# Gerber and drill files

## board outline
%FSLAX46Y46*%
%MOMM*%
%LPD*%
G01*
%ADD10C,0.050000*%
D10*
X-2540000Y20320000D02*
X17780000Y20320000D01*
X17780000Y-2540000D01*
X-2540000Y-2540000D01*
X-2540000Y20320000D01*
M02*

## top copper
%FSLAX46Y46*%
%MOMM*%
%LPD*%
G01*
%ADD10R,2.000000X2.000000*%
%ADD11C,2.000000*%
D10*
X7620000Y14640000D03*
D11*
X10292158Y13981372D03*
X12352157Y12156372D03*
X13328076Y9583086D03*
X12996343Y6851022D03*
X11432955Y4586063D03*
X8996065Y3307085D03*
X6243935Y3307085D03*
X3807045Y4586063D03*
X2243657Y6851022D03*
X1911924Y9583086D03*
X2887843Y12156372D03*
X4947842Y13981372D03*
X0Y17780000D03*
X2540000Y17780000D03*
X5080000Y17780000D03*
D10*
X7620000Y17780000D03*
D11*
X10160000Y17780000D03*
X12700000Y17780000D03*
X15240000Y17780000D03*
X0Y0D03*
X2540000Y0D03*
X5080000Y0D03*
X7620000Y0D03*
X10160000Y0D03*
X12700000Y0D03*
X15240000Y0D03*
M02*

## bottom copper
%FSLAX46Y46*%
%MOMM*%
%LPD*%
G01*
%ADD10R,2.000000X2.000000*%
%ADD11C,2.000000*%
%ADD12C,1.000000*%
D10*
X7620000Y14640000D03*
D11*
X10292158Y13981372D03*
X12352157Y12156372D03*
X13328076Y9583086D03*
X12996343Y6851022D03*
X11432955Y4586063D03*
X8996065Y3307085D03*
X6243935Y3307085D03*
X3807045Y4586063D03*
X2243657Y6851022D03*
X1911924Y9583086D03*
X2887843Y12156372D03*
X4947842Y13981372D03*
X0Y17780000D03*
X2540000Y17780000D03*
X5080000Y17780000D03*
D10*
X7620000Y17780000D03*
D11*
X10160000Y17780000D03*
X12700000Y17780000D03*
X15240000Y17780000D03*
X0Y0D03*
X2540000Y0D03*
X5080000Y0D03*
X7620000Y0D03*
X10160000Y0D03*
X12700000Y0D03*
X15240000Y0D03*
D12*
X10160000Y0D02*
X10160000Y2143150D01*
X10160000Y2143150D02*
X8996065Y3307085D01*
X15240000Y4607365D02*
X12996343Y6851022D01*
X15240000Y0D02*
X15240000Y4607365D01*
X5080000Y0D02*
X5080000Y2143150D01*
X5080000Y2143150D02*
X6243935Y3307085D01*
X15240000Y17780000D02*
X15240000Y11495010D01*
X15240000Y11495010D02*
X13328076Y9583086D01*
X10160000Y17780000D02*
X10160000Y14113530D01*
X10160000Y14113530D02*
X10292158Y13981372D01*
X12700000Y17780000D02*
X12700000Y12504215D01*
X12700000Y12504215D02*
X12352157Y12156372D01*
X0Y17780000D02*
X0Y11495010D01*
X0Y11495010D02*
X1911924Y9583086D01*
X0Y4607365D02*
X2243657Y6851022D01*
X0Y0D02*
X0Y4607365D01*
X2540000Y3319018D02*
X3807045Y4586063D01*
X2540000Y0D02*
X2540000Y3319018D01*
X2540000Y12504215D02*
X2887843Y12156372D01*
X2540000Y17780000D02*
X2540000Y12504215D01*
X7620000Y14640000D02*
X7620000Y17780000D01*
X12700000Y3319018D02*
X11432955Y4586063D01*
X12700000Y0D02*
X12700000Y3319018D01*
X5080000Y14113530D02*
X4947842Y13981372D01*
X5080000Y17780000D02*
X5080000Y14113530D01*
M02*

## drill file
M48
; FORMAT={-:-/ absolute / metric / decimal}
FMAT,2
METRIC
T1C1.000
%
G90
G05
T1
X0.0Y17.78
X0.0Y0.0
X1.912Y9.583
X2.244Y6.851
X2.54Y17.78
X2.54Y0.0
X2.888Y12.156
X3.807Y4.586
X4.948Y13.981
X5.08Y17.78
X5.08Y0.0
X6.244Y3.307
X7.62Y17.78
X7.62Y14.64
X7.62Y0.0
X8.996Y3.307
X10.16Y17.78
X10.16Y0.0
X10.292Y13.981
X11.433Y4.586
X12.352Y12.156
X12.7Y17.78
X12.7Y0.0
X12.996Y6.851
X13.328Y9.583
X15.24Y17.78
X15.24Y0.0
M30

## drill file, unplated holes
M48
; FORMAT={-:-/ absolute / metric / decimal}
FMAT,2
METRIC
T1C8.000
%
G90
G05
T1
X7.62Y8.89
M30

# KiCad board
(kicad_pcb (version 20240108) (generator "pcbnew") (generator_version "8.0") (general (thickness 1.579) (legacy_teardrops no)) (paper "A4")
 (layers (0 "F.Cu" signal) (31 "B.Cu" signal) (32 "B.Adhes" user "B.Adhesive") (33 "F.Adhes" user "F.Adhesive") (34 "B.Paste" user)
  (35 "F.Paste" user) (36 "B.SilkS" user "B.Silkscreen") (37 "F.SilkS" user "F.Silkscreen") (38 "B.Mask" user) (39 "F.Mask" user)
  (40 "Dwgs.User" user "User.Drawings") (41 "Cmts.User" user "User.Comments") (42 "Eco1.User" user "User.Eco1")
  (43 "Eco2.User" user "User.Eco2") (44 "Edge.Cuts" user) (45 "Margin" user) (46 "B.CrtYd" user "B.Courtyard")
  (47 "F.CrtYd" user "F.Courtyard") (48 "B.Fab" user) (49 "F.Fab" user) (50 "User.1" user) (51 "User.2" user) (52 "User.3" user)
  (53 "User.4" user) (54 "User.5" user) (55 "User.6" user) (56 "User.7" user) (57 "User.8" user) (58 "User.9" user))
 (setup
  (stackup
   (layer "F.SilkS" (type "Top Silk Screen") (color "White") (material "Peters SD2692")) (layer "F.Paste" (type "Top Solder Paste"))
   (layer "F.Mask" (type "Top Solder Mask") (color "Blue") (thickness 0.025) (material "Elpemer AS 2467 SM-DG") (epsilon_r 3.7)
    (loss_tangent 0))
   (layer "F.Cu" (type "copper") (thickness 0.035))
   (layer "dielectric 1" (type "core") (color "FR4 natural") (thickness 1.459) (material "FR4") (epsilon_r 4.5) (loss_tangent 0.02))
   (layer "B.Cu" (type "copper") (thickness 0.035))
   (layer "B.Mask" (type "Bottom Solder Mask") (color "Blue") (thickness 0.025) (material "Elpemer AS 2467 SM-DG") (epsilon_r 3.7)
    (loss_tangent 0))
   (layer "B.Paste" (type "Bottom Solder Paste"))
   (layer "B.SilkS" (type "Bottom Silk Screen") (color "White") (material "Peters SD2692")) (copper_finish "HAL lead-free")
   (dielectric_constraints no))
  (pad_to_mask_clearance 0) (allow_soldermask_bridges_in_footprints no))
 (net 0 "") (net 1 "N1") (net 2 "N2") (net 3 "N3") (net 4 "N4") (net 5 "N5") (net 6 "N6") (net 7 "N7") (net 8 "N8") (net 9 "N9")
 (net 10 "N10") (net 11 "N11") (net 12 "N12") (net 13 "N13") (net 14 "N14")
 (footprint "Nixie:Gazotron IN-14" (layer "F.Cu") (at 7.62 -8.89)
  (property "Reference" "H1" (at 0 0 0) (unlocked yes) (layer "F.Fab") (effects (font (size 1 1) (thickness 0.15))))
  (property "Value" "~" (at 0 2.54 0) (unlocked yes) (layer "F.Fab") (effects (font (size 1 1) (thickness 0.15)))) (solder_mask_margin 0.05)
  (pad "" np_thru_hole circle (at 0 0) (size 2 2) (drill 8) (layers "*.Mask"))
  (pad "1" thru_hole rect (at 0 -5.75) (size 2 2) (drill 1) (layers "*.Cu" "B.Mask") (remove_unused_layers no) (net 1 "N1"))
  (pad "2" thru_hole circle (at 2.672158 -5.091372) (size 2 2) (drill 1) (layers "*.Cu" "B.Mask") (remove_unused_layers no) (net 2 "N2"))
  (pad "3" thru_hole circle (at 4.732157 -3.266372) (size 2 2) (drill 1) (layers "*.Cu" "B.Mask") (remove_unused_layers no) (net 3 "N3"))
  (pad "4" thru_hole circle (at 5.708076 -0.693086) (size 2 2) (drill 1) (layers "*.Cu" "B.Mask") (remove_unused_layers no) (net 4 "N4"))
  (pad "5" thru_hole circle (at 5.376343 2.038978) (size 2 2) (drill 1) (layers "*.Cu" "B.Mask") (remove_unused_layers no) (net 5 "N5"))
  (pad "6" thru_hole circle (at 3.812955 4.303937) (size 2 2) (drill 1) (layers "*.Cu" "B.Mask") (remove_unused_layers no) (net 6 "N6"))
  (pad "7" thru_hole circle (at 1.376065 5.582915) (size 2 2) (drill 1) (layers "*.Cu" "B.Mask") (remove_unused_layers no) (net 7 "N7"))
  (pad "8" thru_hole circle (at -1.376065 5.582915) (size 2 2) (drill 1) (layers "*.Cu" "B.Mask") (remove_unused_layers no) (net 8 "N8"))
  (pad "9" thru_hole circle (at -3.812955 4.303937) (size 2 2) (drill 1) (layers "*.Cu" "B.Mask") (remove_unused_layers no) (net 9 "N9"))
  (pad "10" thru_hole circle (at -5.376343 2.038978) (size 2 2) (drill 1) (layers "*.Cu" "B.Mask") (remove_unused_layers no) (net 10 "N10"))
  (pad "11" thru_hole circle (at -5.708076 -0.693086) (size 2 2) (drill 1) (layers "*.Cu" "B.Mask") (remove_unused_layers no) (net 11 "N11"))
  (pad "12" thru_hole circle (at -4.732157 -3.266372) (size 2 2) (drill 1) (layers "*.Cu" "B.Mask") (remove_unused_layers no) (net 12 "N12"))
  (pad "13" thru_hole circle (at -2.672158 -5.091372) (size 2 2) (drill 1) (layers "*.Cu" "B.Mask") (remove_unused_layers no) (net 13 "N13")))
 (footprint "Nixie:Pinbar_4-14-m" (layer "F.Cu") (at 0 0)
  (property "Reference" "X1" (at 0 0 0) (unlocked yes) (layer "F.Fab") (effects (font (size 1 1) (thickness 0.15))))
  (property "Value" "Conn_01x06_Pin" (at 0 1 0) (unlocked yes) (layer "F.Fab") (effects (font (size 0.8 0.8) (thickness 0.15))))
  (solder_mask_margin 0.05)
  (pad "1" thru_hole circle (at 0 -17.78) (size 2 2) (drill 1) (layers "*.Cu" "F.Mask") (remove_unused_layers no) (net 11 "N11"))
  (pad "2" thru_hole circle (at 2.54 -17.78) (size 2 2) (drill 1) (layers "*.Cu" "F.Mask") (remove_unused_layers no) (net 12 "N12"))
  (pad "3" thru_hole circle (at 5.08 -17.78) (size 2 2) (drill 1) (layers "*.Cu" "F.Mask") (remove_unused_layers no) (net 13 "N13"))
  (pad "4" thru_hole rect (at 7.62 -17.78) (size 2 2) (drill 1) (layers "*.Cu" "F.Mask") (remove_unused_layers no) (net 1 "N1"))
  (pad "5" thru_hole circle (at 10.16 -17.78) (size 2 2) (drill 1) (layers "*.Cu" "F.Mask") (remove_unused_layers no) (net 2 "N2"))
  (pad "6" thru_hole circle (at 12.7 -17.78) (size 2 2) (drill 1) (layers "*.Cu" "F.Mask") (remove_unused_layers no) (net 3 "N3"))
  (pad "7" thru_hole circle (at 15.24 -17.78) (size 2 2) (drill 1) (layers "*.Cu" "F.Mask") (remove_unused_layers no) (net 4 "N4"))
  (pad "8" thru_hole circle (at 0 0) (size 2 2) (drill 1) (layers "*.Cu" "F.Mask") (remove_unused_layers no) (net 10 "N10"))
  (pad "9" thru_hole circle (at 2.54 0) (size 2 2) (drill 1) (layers "*.Cu" "F.Mask") (remove_unused_layers no) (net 9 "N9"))
  (pad "10" thru_hole circle (at 5.08 0) (size 2 2) (drill 1) (layers "*.Cu" "F.Mask") (remove_unused_layers no) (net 8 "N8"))
  (pad "11" thru_hole circle (at 7.62 0) (size 2 2) (drill 1) (layers "*.Cu" "F.Mask") (remove_unused_layers no) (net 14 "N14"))
  (pad "12" thru_hole circle (at 10.16 0) (size 2 2) (drill 1) (layers "*.Cu" "F.Mask") (remove_unused_layers no) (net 7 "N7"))
  (pad "13" thru_hole circle (at 12.7 0) (size 2 2) (drill 1) (layers "*.Cu" "F.Mask") (remove_unused_layers no) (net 6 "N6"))
  (pad "14" thru_hole circle (at 15.24 0) (size 2 2) (drill 1) (layers "*.Cu" "F.Mask") (remove_unused_layers no) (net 5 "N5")))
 (gr_rect (start -2.54 -20.32) (end 17.78 2.54) (stroke (width 0.05) (type default)) (fill none) (layer "Edge.Cuts"))
 (segment (start 10.16 0) (end 10.16 -2.14315) (width 1) (layer "B.Cu") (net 7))
 (segment (start 10.16 -2.14315) (end 8.996065 -3.307085) (width 1) (layer "B.Cu") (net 7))
 (segment (start 15.24 -4.607365) (end 12.996343 -6.851022) (width 1) (layer "B.Cu") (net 5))
 (segment (start 15.24 0) (end 15.24 -4.607365) (width 1) (layer "B.Cu") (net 5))
 (segment (start 5.08 0) (end 5.08 -2.14315) (width 1) (layer "B.Cu") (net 8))
 (segment (start 5.08 -2.14315) (end 6.243935 -3.307085) (width 1) (layer "B.Cu") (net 8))
 (segment (start 15.24 -17.78) (end 15.24 -11.49501) (width 1) (layer "B.Cu") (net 4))
 (segment (start 15.24 -11.49501) (end 13.328076 -9.583086) (width 1) (layer "B.Cu") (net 4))
 (segment (start 10.16 -17.78) (end 10.16 -14.11353) (width 1) (layer "B.Cu") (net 2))
 (segment (start 10.16 -14.11353) (end 10.292158 -13.981372) (width 1) (layer "B.Cu") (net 2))
 (segment (start 12.7 -17.78) (end 12.7 -12.504215) (width 1) (layer "B.Cu") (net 3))
 (segment (start 12.7 -12.504215) (end 12.352157 -12.156372) (width 1) (layer "B.Cu") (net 3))
 (segment (start 0 -17.78) (end 0 -11.49501) (width 1) (layer "B.Cu") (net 11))
 (segment (start 0 -11.49501) (end 1.911924 -9.583086) (width 1) (layer "B.Cu") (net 11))
 (segment (start 0 -4.607365) (end 2.243657 -6.851022) (width 1) (layer "B.Cu") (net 10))
 (segment (start 0 0) (end 0 -4.607365) (width 1) (layer "B.Cu") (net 10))
 (segment (start 2.54 -3.319018) (end 3.807045 -4.586063) (width 1) (layer "B.Cu") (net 9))
 (segment (start 2.54 0) (end 2.54 -3.319018) (width 1) (layer "B.Cu") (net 9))
 (segment (start 2.54 -12.504215) (end 2.887843 -12.156372) (width 1) (layer "B.Cu") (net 12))
 (segment (start 2.54 -17.78) (end 2.54 -12.504215) (width 1) (layer "B.Cu") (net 12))
 (segment (start 7.62 -14.64) (end 7.62 -17.78) (width 1) (layer "B.Cu") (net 1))
 (segment (start 12.7 -3.319018) (end 11.432955 -4.586063) (width 1) (layer "B.Cu") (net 6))
 (segment (start 12.7 0) (end 12.7 -3.319018) (width 1) (layer "B.Cu") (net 6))
 (segment (start 5.08 -14.11353) (end 4.947842 -13.981372) (width 1) (layer "B.Cu") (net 13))
 (segment (start 5.08 -17.78) (end 5.08 -14.11353) (width 1) (layer "B.Cu") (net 13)))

